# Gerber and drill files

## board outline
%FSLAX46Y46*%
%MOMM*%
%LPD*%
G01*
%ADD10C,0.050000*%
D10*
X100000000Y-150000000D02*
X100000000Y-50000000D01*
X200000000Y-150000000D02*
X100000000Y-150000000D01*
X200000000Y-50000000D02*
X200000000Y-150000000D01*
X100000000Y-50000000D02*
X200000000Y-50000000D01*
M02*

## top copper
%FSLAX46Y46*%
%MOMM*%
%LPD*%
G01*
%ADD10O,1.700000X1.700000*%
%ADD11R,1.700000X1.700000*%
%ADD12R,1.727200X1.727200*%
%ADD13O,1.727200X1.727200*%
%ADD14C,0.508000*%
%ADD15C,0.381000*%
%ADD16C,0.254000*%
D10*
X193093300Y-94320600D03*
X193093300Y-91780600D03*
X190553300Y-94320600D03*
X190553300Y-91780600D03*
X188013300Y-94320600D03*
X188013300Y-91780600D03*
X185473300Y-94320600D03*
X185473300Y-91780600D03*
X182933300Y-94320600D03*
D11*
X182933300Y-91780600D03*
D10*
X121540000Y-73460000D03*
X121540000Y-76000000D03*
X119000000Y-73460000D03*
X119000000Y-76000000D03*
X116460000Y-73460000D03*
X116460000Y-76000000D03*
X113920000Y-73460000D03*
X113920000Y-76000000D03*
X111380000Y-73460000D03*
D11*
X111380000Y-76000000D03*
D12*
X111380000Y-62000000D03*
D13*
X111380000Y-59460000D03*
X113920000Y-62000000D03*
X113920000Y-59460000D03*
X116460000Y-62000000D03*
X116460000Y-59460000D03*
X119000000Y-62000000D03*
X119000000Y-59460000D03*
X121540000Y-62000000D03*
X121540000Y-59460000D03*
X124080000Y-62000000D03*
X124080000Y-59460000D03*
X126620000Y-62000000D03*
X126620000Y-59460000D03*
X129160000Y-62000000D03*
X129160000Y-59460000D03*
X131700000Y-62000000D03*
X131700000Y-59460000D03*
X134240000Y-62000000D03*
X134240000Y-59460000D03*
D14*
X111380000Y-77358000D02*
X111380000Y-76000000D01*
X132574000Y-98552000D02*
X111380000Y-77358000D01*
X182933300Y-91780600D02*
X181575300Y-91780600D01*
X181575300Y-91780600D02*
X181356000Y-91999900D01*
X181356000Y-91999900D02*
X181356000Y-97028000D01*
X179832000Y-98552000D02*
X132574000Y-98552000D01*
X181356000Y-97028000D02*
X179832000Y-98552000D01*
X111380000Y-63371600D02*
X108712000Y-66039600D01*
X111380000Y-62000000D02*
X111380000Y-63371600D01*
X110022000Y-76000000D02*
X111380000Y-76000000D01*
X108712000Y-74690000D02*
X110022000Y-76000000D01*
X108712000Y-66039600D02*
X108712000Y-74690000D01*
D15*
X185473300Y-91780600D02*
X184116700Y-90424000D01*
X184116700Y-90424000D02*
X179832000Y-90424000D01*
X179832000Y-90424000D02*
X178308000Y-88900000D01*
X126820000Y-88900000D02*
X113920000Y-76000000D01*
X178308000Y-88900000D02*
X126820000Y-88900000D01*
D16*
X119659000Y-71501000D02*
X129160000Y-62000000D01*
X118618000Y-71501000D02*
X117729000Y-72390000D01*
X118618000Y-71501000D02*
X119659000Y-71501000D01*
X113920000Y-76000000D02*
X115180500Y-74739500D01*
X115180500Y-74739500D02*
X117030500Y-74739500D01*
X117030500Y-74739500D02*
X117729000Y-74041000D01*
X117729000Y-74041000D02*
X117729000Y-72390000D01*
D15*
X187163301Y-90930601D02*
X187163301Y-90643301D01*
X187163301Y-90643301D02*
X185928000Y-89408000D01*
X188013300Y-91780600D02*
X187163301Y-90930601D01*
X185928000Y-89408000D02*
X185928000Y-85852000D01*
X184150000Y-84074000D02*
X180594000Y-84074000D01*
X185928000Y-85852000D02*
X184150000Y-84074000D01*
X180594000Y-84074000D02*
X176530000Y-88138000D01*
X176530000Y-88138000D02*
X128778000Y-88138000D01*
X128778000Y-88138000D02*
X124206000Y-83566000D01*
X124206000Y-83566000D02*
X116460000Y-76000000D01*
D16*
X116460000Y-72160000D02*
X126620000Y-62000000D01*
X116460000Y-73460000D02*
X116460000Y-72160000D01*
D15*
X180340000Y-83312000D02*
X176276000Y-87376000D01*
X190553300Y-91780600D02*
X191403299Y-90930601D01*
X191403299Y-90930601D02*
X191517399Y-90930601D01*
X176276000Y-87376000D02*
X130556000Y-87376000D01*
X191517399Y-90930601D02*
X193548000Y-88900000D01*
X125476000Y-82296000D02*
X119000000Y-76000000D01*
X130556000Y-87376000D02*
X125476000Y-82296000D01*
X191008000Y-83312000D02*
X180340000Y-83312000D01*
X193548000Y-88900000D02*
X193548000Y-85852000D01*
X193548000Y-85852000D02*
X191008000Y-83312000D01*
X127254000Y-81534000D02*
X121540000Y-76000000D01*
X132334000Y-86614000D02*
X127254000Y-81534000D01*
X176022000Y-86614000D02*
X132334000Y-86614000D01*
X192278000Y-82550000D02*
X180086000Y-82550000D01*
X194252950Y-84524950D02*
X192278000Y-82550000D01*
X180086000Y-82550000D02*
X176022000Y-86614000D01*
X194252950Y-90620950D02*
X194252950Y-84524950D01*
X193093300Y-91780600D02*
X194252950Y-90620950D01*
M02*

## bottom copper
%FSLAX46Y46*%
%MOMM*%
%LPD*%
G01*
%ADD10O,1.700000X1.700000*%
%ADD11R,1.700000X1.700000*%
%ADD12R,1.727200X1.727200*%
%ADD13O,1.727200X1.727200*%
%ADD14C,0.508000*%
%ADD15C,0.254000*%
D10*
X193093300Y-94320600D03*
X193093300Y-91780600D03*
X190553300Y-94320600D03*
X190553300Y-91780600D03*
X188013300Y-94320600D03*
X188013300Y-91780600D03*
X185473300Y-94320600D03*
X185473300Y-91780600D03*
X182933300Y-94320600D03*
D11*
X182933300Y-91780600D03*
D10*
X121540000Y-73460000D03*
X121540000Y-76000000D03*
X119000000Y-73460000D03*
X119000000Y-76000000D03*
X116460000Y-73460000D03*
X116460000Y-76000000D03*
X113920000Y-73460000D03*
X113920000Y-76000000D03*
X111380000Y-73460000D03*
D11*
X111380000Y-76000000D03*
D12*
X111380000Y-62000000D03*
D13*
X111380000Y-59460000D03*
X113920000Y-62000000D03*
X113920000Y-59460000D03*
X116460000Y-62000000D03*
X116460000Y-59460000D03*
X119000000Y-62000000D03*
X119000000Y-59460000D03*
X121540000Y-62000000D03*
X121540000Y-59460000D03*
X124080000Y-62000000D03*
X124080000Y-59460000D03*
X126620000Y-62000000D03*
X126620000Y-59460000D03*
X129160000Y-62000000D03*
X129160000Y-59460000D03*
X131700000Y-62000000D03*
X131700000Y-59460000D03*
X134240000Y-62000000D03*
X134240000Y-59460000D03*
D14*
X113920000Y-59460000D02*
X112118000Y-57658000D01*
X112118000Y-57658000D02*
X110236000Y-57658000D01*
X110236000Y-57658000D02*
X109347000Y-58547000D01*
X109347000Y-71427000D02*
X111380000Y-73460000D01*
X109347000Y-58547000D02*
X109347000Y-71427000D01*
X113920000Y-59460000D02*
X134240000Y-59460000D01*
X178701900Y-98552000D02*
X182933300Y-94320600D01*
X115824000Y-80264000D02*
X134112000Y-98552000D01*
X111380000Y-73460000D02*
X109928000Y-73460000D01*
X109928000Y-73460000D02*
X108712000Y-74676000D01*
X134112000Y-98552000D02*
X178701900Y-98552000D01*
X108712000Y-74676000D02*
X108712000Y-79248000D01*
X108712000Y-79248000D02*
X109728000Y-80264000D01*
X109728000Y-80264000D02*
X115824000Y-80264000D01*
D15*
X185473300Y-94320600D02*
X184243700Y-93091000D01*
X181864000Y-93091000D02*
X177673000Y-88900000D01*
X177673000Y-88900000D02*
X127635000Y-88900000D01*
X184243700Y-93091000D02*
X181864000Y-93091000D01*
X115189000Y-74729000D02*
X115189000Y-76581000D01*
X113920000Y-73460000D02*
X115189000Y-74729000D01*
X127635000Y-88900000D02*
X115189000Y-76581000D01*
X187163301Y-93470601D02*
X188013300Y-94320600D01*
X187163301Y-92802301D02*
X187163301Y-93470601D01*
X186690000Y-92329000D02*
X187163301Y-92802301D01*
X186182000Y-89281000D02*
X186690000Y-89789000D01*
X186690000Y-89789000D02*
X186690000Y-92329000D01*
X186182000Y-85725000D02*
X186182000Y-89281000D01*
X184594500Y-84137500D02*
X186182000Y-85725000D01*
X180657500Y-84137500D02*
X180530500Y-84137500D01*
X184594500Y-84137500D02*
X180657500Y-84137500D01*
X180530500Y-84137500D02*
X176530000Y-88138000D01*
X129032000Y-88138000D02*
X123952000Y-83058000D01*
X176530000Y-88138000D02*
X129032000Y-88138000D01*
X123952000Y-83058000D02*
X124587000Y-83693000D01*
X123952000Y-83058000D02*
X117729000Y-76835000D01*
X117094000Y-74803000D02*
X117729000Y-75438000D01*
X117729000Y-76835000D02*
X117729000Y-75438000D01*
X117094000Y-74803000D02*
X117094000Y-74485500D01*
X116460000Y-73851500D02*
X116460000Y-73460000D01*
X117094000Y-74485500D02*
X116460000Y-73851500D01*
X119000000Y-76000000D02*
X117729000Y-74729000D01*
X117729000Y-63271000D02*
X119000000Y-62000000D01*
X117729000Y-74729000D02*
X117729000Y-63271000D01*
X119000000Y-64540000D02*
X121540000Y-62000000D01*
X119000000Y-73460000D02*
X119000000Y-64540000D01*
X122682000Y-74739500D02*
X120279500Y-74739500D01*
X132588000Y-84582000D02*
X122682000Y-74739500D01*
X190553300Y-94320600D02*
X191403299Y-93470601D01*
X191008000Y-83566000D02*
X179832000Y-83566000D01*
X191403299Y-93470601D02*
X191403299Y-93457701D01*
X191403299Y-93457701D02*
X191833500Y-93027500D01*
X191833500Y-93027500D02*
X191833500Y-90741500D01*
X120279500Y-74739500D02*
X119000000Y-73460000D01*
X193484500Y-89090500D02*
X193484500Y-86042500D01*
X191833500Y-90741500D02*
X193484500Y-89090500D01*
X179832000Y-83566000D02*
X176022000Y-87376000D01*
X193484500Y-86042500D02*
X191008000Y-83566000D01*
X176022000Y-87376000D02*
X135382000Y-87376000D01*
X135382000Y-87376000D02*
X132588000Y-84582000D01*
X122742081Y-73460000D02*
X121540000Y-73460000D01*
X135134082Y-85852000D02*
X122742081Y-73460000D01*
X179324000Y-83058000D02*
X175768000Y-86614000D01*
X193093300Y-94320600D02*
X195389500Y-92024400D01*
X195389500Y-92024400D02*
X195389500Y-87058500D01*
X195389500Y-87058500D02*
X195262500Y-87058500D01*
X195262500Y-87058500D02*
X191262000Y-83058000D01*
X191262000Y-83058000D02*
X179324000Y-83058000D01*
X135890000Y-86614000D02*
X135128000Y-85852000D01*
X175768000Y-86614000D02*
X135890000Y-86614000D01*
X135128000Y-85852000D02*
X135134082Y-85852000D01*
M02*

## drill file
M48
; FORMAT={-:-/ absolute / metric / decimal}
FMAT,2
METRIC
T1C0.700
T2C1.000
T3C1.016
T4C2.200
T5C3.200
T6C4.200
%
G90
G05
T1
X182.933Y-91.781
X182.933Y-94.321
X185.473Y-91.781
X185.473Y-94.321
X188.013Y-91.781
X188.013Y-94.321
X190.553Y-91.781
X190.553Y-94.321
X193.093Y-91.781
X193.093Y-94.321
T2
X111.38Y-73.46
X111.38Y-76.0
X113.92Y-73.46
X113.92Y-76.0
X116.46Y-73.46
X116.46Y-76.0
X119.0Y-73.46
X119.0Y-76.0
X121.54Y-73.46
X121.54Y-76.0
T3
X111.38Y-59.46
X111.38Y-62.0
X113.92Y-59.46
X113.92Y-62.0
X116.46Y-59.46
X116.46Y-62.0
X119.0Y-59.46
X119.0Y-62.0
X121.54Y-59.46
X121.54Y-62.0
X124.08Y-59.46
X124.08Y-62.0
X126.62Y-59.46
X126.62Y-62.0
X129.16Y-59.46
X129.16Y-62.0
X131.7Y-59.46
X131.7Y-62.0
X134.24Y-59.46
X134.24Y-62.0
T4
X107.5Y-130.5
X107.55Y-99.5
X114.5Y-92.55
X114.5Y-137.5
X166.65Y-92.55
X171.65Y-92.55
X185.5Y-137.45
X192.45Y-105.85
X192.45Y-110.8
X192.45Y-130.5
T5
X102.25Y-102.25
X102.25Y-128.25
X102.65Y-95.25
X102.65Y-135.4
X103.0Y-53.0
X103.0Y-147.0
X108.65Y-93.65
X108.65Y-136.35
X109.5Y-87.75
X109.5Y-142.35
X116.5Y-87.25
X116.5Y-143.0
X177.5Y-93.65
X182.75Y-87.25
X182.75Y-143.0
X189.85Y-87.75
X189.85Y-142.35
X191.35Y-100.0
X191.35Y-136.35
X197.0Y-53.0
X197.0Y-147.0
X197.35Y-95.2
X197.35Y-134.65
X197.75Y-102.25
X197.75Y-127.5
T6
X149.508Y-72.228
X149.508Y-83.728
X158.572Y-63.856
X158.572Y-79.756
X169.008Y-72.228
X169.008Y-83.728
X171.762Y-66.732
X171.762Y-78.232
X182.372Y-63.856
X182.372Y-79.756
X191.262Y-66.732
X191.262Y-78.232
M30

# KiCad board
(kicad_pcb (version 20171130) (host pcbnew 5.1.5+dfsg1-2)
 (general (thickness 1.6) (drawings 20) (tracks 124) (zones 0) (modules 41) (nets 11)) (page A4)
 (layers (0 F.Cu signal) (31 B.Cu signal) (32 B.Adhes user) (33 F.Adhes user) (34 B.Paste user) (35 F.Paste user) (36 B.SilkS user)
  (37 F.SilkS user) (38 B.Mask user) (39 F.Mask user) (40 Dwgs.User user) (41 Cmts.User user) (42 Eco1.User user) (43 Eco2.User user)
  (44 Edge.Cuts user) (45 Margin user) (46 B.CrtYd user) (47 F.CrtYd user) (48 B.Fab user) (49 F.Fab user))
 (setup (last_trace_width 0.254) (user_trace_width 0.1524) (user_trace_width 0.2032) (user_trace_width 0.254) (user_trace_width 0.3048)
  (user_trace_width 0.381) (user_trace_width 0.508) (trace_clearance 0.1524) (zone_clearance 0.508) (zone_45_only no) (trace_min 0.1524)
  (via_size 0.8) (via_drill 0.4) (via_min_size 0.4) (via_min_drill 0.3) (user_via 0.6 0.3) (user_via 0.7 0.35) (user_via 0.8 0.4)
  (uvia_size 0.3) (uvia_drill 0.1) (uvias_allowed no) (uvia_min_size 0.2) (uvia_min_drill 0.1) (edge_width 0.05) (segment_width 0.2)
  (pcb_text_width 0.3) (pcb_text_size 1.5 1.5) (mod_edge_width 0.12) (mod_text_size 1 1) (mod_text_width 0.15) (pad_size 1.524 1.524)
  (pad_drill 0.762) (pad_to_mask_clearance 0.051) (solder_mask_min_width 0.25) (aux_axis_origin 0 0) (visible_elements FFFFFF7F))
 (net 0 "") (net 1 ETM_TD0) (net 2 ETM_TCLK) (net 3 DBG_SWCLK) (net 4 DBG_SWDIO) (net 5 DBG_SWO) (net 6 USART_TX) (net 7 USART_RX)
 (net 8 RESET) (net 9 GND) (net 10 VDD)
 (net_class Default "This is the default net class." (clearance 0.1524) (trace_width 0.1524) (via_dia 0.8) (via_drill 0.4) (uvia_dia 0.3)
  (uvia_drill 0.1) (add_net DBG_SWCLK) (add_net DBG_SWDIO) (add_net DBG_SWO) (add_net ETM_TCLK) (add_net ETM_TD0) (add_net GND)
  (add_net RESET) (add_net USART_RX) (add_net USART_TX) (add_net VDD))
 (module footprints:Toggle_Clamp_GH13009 (layer F.Cu) (at 181.512 72.482)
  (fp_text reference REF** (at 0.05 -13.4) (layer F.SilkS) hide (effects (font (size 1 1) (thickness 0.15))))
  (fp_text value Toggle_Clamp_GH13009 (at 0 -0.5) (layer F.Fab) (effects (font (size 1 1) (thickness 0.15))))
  (pad "" np_thru_hole circle (at -9.75 -5.75) (size 4.2 4.2) (drill 4.2) (layers *.Cu *.Mask))
  (pad "" np_thru_hole circle (at -9.75 5.75) (size 4.2 4.2) (drill 4.2) (layers *.Cu *.Mask))
  (pad "" np_thru_hole circle (at 9.75 5.75) (size 4.2 4.2) (drill 4.2) (layers *.Cu *.Mask))
  (pad "" np_thru_hole circle (at 9.75 -5.75) (size 4.2 4.2) (drill 4.2) (layers *.Cu *.Mask)))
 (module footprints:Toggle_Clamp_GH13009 (layer F.Cu) (at 159.258 77.978)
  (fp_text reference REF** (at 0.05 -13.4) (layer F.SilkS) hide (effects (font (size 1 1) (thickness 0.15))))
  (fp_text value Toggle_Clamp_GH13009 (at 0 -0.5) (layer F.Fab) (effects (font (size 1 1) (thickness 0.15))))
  (pad "" np_thru_hole circle (at 9.75 -5.75) (size 4.2 4.2) (drill 4.2) (layers *.Cu *.Mask))
  (pad "" np_thru_hole circle (at 9.75 5.75) (size 4.2 4.2) (drill 4.2) (layers *.Cu *.Mask))
  (pad "" np_thru_hole circle (at -9.75 5.75) (size 4.2 4.2) (drill 4.2) (layers *.Cu *.Mask))
  (pad "" np_thru_hole circle (at -9.75 -5.75) (size 4.2 4.2) (drill 4.2) (layers *.Cu *.Mask)))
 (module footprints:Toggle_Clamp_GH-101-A (layer F.Cu) (at 170.472 71.806)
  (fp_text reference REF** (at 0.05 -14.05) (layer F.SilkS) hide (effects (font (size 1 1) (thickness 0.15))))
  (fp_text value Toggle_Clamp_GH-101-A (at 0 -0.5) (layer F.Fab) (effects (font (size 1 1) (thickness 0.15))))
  (pad "" np_thru_hole circle (at -11.9 -7.95) (size 4.2 4.2) (drill 4.2) (layers *.Cu *.Mask))
  (pad "" np_thru_hole circle (at -11.9 7.95) (size 4.2 4.2) (drill 4.2) (layers *.Cu *.Mask))
  (pad "" np_thru_hole circle (at 11.9 7.95) (size 4.2 4.2) (drill 4.2) (layers *.Cu *.Mask))
  (pad "" np_thru_hole circle (at 11.9 -7.95) (size 4.2 4.2) (drill 4.2) (layers *.Cu *.Mask)))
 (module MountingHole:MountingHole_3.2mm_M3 (layer F.Cu) (at 197 53)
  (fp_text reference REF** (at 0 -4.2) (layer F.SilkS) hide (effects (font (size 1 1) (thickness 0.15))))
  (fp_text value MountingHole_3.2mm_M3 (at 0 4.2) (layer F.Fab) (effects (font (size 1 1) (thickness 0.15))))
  (pad 1 np_thru_hole circle (at 0 0) (size 3.2 3.2) (drill 3.2) (layers *.Cu *.Mask)))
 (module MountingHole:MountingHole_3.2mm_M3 (layer F.Cu) (at 197 147)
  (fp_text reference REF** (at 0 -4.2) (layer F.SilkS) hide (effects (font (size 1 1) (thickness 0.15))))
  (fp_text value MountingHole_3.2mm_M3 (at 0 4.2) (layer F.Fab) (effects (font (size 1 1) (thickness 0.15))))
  (pad 1 np_thru_hole circle (at 0 0) (size 3.2 3.2) (drill 3.2) (layers *.Cu *.Mask)))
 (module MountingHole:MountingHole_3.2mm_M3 (layer F.Cu) (at 103 147)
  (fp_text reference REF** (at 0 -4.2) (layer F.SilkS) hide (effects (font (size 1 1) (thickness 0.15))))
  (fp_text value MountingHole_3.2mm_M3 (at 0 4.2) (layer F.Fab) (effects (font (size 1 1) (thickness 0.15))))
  (pad 1 np_thru_hole circle (at 0 0) (size 3.2 3.2) (drill 3.2) (layers *.Cu *.Mask)))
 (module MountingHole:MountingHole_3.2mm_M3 (layer F.Cu) (at 103 53)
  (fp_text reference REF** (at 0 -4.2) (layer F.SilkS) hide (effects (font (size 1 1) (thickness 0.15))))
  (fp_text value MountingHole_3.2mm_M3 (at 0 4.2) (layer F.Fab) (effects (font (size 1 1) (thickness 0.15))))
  (pad 1 np_thru_hole circle (at 0 0) (size 3.2 3.2) (drill 3.2) (layers *.Cu *.Mask)))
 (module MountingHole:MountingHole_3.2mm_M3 (layer F.Cu) (at 116.5 87.25)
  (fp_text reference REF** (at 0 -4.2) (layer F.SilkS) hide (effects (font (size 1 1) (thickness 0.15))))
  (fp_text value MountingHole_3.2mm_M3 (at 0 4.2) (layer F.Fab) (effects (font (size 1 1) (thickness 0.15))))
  (pad 1 np_thru_hole circle (at 0 0) (size 3.2 3.2) (drill 3.2) (layers *.Cu *.Mask)))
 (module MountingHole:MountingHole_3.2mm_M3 (layer F.Cu) (at 102.25 102.25)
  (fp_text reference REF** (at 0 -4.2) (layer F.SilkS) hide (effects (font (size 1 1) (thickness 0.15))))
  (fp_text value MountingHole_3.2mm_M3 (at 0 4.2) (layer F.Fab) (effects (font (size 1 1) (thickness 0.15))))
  (pad 1 np_thru_hole circle (at 0 0) (size 3.2 3.2) (drill 3.2) (layers *.Cu *.Mask)))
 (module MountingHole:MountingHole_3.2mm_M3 (layer F.Cu) (at 102.25 128.25)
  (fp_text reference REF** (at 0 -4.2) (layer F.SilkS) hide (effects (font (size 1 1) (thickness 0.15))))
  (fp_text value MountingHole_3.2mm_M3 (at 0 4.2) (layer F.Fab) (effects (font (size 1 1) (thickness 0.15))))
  (pad 1 np_thru_hole circle (at 0 0) (size 3.2 3.2) (drill 3.2) (layers *.Cu *.Mask)))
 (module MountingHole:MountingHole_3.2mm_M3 (layer F.Cu) (at 116.5 143)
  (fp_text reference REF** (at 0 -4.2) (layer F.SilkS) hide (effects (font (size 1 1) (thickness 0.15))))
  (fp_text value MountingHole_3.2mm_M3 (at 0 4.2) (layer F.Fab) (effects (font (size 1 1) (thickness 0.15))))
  (pad 1 np_thru_hole circle (at 0 0) (size 3.2 3.2) (drill 3.2) (layers *.Cu *.Mask)))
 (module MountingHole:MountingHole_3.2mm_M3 (layer F.Cu) (at 182.75 143)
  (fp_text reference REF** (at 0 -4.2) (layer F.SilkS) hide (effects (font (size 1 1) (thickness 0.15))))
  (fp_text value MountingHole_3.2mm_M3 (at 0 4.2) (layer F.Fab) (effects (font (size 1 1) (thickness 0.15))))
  (pad 1 np_thru_hole circle (at 0 0) (size 3.2 3.2) (drill 3.2) (layers *.Cu *.Mask)))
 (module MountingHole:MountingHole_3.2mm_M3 (layer F.Cu) (at 197.75 127.5)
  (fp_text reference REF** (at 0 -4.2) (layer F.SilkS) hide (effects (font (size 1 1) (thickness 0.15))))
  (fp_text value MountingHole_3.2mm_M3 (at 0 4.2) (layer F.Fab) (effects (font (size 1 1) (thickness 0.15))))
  (pad 1 np_thru_hole circle (at 0 0) (size 3.2 3.2) (drill 3.2) (layers *.Cu *.Mask)))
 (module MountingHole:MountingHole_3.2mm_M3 (layer F.Cu) (at 182.75 87.25)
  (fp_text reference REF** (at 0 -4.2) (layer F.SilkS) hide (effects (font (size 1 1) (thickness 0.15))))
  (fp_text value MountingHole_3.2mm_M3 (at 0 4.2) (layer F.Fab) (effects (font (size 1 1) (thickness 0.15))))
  (pad 1 np_thru_hole circle (at 0 0) (size 3.2 3.2) (drill 3.2) (layers *.Cu *.Mask)))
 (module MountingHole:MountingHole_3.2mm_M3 (layer F.Cu) (at 197.75 102.25)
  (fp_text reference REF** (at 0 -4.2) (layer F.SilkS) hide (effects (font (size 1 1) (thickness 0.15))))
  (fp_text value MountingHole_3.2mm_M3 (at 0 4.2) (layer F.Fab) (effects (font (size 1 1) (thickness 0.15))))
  (pad 1 np_thru_hole circle (at 0 0) (size 3.2 3.2) (drill 3.2) (layers *.Cu *.Mask)))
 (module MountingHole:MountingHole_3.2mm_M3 (layer F.Cu) (at 102.65 95.25)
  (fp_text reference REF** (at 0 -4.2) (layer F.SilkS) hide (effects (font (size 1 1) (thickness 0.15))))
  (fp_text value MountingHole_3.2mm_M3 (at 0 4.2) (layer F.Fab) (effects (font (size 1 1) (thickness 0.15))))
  (pad 1 np_thru_hole circle (at 0 0) (size 3.2 3.2) (drill 3.2) (layers *.Cu *.Mask)))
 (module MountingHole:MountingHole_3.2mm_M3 (layer F.Cu) (at 109.5 87.75)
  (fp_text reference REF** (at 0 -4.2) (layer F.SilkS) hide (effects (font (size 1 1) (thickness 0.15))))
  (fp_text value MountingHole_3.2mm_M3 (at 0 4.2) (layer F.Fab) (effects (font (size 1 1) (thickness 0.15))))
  (pad 1 np_thru_hole circle (at 0 0) (size 3.2 3.2) (drill 3.2) (layers *.Cu *.Mask)))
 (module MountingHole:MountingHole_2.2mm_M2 (layer F.Cu) (at 192.45 110.8)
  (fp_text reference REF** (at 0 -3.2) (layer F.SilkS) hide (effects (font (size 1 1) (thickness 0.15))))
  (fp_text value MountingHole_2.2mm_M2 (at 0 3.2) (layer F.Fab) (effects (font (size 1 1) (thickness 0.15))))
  (pad 1 np_thru_hole circle (at 0 0) (size 2.2 2.2) (drill 2.2) (layers *.Cu *.Mask)))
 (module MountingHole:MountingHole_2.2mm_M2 (layer F.Cu) (at 166.65 92.55)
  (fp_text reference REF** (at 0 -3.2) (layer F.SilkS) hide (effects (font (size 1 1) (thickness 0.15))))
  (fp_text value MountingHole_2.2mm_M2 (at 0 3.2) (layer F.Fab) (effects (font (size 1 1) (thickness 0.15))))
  (pad 1 np_thru_hole circle (at 0 0) (size 2.2 2.2) (drill 2.2) (layers *.Cu *.Mask)))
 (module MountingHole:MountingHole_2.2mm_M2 (layer F.Cu) (at 171.65 92.55)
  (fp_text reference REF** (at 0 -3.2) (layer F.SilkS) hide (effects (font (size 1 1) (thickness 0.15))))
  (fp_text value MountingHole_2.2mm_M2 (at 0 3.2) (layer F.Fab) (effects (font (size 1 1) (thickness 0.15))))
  (pad 1 np_thru_hole circle (at 0 0) (size 2.2 2.2) (drill 2.2) (layers *.Cu *.Mask)))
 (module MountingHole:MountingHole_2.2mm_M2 (layer F.Cu) (at 192.45 105.85)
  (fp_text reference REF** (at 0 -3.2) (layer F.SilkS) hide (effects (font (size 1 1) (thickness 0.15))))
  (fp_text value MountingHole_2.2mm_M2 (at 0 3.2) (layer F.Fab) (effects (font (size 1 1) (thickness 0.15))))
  (pad 1 np_thru_hole circle (at 0 0) (size 2.2 2.2) (drill 2.2) (layers *.Cu *.Mask)))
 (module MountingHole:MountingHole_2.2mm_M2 (layer F.Cu) (at 192.45 130.5)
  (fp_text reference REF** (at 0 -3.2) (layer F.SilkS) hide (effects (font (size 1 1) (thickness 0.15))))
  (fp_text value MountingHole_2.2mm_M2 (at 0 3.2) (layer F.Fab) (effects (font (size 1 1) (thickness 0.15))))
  (pad 1 np_thru_hole circle (at 0 0) (size 2.2 2.2) (drill 2.2) (layers *.Cu *.Mask)))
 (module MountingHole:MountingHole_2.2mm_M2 (layer F.Cu) (at 185.5 137.45)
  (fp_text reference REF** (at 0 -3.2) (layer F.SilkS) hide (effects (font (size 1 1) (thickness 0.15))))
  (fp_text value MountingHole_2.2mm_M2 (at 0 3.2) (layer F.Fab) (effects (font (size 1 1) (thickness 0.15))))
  (pad 1 np_thru_hole circle (at 0 0) (size 2.2 2.2) (drill 2.2) (layers *.Cu *.Mask)))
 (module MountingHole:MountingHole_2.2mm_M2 (layer F.Cu) (at 107.5 130.5)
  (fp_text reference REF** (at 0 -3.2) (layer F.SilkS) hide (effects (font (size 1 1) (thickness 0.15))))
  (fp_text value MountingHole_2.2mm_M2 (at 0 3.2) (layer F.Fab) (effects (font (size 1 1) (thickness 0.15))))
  (pad 1 np_thru_hole circle (at 0 0) (size 2.2 2.2) (drill 2.2) (layers *.Cu *.Mask)))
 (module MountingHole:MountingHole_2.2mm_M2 (layer F.Cu) (at 114.5 137.5)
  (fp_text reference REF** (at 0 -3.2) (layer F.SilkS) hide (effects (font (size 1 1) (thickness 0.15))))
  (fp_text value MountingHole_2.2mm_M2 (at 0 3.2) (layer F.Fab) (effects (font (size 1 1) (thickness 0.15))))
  (pad 1 np_thru_hole circle (at 0 0) (size 2.2 2.2) (drill 2.2) (layers *.Cu *.Mask)))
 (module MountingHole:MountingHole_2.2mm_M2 (layer F.Cu) (at 114.5 92.55)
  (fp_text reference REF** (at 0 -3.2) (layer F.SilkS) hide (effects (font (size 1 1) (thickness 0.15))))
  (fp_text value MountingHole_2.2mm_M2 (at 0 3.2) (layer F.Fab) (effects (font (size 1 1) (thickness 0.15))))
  (pad 1 np_thru_hole circle (at 0 0) (size 2.2 2.2) (drill 2.2) (layers *.Cu *.Mask)))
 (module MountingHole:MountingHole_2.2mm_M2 (layer F.Cu) (at 107.55 99.5)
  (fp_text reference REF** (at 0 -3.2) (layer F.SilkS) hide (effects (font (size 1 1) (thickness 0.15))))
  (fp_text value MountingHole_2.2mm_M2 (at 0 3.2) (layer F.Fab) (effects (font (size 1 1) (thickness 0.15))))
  (pad 1 np_thru_hole circle (at 0 0) (size 2.2 2.2) (drill 2.2) (layers *.Cu *.Mask)))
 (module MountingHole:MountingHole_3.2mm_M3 (layer F.Cu) (at 197.35 95.2)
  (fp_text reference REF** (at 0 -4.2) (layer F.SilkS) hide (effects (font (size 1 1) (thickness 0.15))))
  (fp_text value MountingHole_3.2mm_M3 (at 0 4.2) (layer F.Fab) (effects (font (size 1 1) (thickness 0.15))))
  (pad 1 np_thru_hole circle (at 0 0) (size 3.2 3.2) (drill 3.2) (layers *.Cu *.Mask)))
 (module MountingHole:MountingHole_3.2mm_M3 (layer F.Cu) (at 189.85 87.75)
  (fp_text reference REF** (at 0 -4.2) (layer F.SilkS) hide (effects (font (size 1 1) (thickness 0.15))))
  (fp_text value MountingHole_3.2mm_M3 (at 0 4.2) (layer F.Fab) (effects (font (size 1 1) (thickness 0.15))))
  (pad 1 np_thru_hole circle (at 0 0) (size 3.2 3.2) (drill 3.2) (layers *.Cu *.Mask)))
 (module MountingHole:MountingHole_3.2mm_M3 (layer F.Cu) (at 197.35 134.65)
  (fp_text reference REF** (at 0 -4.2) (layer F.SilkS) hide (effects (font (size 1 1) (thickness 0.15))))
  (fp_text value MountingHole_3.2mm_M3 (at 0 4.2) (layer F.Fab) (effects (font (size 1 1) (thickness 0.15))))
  (pad 1 np_thru_hole circle (at 0 0) (size 3.2 3.2) (drill 3.2) (layers *.Cu *.Mask)))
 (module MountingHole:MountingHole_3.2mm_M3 (layer F.Cu) (at 189.85 142.35)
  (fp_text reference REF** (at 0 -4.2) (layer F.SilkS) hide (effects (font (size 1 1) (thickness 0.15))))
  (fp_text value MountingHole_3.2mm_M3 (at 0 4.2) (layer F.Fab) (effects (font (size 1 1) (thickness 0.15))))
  (pad 1 np_thru_hole circle (at 0 0) (size 3.2 3.2) (drill 3.2) (layers *.Cu *.Mask)))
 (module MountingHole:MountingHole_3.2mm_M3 (layer F.Cu) (at 109.5 142.35)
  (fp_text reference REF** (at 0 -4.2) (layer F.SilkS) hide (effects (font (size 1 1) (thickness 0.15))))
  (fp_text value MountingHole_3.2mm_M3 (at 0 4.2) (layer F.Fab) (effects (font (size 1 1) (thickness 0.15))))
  (pad 1 np_thru_hole circle (at 0 0) (size 3.2 3.2) (drill 3.2) (layers *.Cu *.Mask)))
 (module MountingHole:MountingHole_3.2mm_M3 (layer F.Cu) (at 191.35 100)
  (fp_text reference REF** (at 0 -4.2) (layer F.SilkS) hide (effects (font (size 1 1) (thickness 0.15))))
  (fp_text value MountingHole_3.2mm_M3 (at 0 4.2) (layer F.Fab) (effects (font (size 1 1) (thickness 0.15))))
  (pad 1 np_thru_hole circle (at 0 0) (size 3.2 3.2) (drill 3.2) (layers *.Cu *.Mask)))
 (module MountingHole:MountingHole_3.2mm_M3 (layer F.Cu) (at 191.35 136.35)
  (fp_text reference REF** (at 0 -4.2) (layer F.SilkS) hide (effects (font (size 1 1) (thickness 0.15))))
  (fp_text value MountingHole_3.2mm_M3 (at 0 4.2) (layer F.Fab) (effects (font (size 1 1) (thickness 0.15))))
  (pad 1 np_thru_hole circle (at 0 0) (size 3.2 3.2) (drill 3.2) (layers *.Cu *.Mask)))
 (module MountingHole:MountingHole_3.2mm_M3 (layer F.Cu) (at 177.5 93.65)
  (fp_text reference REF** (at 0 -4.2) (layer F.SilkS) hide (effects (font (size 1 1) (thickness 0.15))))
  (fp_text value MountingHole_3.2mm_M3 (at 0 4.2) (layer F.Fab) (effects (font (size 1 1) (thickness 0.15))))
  (pad 1 np_thru_hole circle (at 0 0) (size 3.2 3.2) (drill 3.2) (layers *.Cu *.Mask)))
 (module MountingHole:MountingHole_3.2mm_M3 (layer F.Cu) (at 108.65 93.65)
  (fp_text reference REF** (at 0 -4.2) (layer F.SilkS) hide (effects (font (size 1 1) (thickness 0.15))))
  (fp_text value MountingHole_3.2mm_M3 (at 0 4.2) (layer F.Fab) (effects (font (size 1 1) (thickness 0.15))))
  (pad 1 np_thru_hole circle (at 0 0) (size 3.2 3.2) (drill 3.2) (layers *.Cu *.Mask)))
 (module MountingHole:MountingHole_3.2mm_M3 (layer F.Cu) (at 102.65 135.4)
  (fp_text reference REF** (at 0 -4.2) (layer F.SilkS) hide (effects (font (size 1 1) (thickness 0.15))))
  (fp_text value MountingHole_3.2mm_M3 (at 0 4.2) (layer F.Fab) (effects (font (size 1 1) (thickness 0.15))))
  (pad 1 np_thru_hole circle (at 0 0) (size 3.2 3.2) (drill 3.2) (layers *.Cu *.Mask)))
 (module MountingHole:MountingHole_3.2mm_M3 (layer F.Cu) (at 108.65 136.35)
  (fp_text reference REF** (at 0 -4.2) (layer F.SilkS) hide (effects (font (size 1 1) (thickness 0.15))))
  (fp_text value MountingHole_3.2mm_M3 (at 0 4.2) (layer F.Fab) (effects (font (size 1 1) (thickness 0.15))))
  (pad 1 np_thru_hole circle (at 0 0) (size 3.2 3.2) (drill 3.2) (layers *.Cu *.Mask)))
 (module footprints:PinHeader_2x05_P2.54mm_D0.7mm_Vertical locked (layer F.Cu) (at 182.9333 94.3206 90)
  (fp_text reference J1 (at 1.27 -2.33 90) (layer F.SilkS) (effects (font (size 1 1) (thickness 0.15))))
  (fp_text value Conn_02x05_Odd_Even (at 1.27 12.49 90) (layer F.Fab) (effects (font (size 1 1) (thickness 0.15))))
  (pad 10 thru_hole oval (at 0 10.16 90) (size 1.7 1.7) (drill 0.7) (layers *.Cu *.Mask) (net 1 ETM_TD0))
  (pad 9 thru_hole oval (at 2.54 10.16 90) (size 1.7 1.7) (drill 0.7) (layers *.Cu *.Mask) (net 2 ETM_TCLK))
  (pad 8 thru_hole oval (at 0 7.62 90) (size 1.7 1.7) (drill 0.7) (layers *.Cu *.Mask) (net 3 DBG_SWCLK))
  (pad 7 thru_hole oval (at 2.54 7.62 90) (size 1.7 1.7) (drill 0.7) (layers *.Cu *.Mask) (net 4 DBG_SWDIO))
  (pad 6 thru_hole oval (at 0 5.08 90) (size 1.7 1.7) (drill 0.7) (layers *.Cu *.Mask) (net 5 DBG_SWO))
  (pad 5 thru_hole oval (at 2.54 5.08 90) (size 1.7 1.7) (drill 0.7) (layers *.Cu *.Mask) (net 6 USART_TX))
  (pad 4 thru_hole oval (at 0 2.54 90) (size 1.7 1.7) (drill 0.7) (layers *.Cu *.Mask) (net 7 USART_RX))
  (pad 3 thru_hole oval (at 2.54 2.54 90) (size 1.7 1.7) (drill 0.7) (layers *.Cu *.Mask) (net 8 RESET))
  (pad 2 thru_hole oval (at 0 0 90) (size 1.7 1.7) (drill 0.7) (layers *.Cu *.Mask) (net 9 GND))
  (pad 1 thru_hole rect (at 2.54 0 90) (size 1.7 1.7) (drill 0.7) (layers *.Cu *.Mask) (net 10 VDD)))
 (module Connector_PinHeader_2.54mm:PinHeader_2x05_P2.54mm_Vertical (layer F.Cu) (at 111.38 76 90)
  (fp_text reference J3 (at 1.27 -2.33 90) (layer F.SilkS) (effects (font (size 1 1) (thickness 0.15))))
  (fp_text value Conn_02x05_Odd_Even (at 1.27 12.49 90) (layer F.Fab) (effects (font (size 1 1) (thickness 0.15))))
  (pad 10 thru_hole oval (at 2.54 10.16 90) (size 1.7 1.7) (drill 1) (layers *.Cu *.Mask) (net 1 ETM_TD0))
  (pad 9 thru_hole oval (at 0 10.16 90) (size 1.7 1.7) (drill 1) (layers *.Cu *.Mask) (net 2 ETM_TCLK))
  (pad 8 thru_hole oval (at 2.54 7.62 90) (size 1.7 1.7) (drill 1) (layers *.Cu *.Mask) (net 3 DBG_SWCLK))
  (pad 7 thru_hole oval (at 0 7.62 90) (size 1.7 1.7) (drill 1) (layers *.Cu *.Mask) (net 4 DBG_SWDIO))
  (pad 6 thru_hole oval (at 2.54 5.08 90) (size 1.7 1.7) (drill 1) (layers *.Cu *.Mask) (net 5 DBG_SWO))
  (pad 5 thru_hole oval (at 0 5.08 90) (size 1.7 1.7) (drill 1) (layers *.Cu *.Mask) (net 6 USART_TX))
  (pad 4 thru_hole oval (at 2.54 2.54 90) (size 1.7 1.7) (drill 1) (layers *.Cu *.Mask) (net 7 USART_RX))
  (pad 3 thru_hole oval (at 0 2.54 90) (size 1.7 1.7) (drill 1) (layers *.Cu *.Mask) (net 8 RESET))
  (pad 2 thru_hole oval (at 2.54 0 90) (size 1.7 1.7) (drill 1) (layers *.Cu *.Mask) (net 9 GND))
  (pad 1 thru_hole rect (at 0 0 90) (size 1.7 1.7) (drill 1) (layers *.Cu *.Mask) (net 10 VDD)))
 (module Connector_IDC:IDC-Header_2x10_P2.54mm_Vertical (layer F.Cu) (at 111.38 62 90)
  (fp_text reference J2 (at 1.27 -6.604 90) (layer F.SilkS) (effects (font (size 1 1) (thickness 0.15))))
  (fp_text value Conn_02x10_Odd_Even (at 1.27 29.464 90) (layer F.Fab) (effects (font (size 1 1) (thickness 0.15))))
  (pad 1 thru_hole rect (at 0 0 90) (size 1.7272 1.7272) (drill 1.016) (layers *.Cu *.Mask) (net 10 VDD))
  (pad 2 thru_hole oval (at 2.54 0 90) (size 1.7272 1.7272) (drill 1.016) (layers *.Cu *.Mask))
  (pad 3 thru_hole oval (at 0 2.54 90) (size 1.7272 1.7272) (drill 1.016) (layers *.Cu *.Mask))
  (pad 4 thru_hole oval (at 2.54 2.54 90) (size 1.7272 1.7272) (drill 1.016) (layers *.Cu *.Mask) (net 9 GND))
  (pad 5 thru_hole oval (at 0 5.08 90) (size 1.7272 1.7272) (drill 1.016) (layers *.Cu *.Mask))
  (pad 6 thru_hole oval (at 2.54 5.08 90) (size 1.7272 1.7272) (drill 1.016) (layers *.Cu *.Mask) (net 9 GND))
  (pad 7 thru_hole oval (at 0 7.62 90) (size 1.7272 1.7272) (drill 1.016) (layers *.Cu *.Mask) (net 4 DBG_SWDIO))
  (pad 8 thru_hole oval (at 2.54 7.62 90) (size 1.7272 1.7272) (drill 1.016) (layers *.Cu *.Mask) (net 9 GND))
  (pad 9 thru_hole oval (at 0 10.16 90) (size 1.7272 1.7272) (drill 1.016) (layers *.Cu *.Mask) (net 3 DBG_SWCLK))
  (pad 10 thru_hole oval (at 2.54 10.16 90) (size 1.7272 1.7272) (drill 1.016) (layers *.Cu *.Mask) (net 9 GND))
  (pad 11 thru_hole oval (at 0 12.7 90) (size 1.7272 1.7272) (drill 1.016) (layers *.Cu *.Mask))
  (pad 12 thru_hole oval (at 2.54 12.7 90) (size 1.7272 1.7272) (drill 1.016) (layers *.Cu *.Mask) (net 9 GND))
  (pad 13 thru_hole oval (at 0 15.24 90) (size 1.7272 1.7272) (drill 1.016) (layers *.Cu *.Mask) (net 5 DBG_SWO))
  (pad 14 thru_hole oval (at 2.54 15.24 90) (size 1.7272 1.7272) (drill 1.016) (layers *.Cu *.Mask) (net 9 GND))
  (pad 15 thru_hole oval (at 0 17.78 90) (size 1.7272 1.7272) (drill 1.016) (layers *.Cu *.Mask) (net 8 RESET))
  (pad 16 thru_hole oval (at 2.54 17.78 90) (size 1.7272 1.7272) (drill 1.016) (layers *.Cu *.Mask) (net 9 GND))
  (pad 17 thru_hole oval (at 0 20.32 90) (size 1.7272 1.7272) (drill 1.016) (layers *.Cu *.Mask))
  (pad 18 thru_hole oval (at 2.54 20.32 90) (size 1.7272 1.7272) (drill 1.016) (layers *.Cu *.Mask) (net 9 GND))
  (pad 19 thru_hole oval (at 0 22.86 90) (size 1.7272 1.7272) (drill 1.016) (layers *.Cu *.Mask))
  (pad 20 thru_hole oval (at 2.54 22.86 90) (size 1.7272 1.7272) (drill 1.016) (layers *.Cu *.Mask) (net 9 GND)))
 (gr_line (start 100 150) (end 100 50) (layer Edge.Cuts) (width 0.05))
 (gr_line (start 200 150) (end 100 150) (layer Edge.Cuts) (width 0.05))
 (gr_line (start 200 50) (end 200 150) (layer Edge.Cuts) (width 0.05))
 (gr_line (start 100 50) (end 200 50) (layer Edge.Cuts) (width 0.05))
 (segment (start 111.38 77.358) (end 111.38 76) (width 0.508) (layer F.Cu) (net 10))
 (segment (start 132.574 98.552) (end 111.38 77.358) (width 0.508) (layer F.Cu) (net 10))
 (segment (start 182.9333 91.7806) (end 181.5753 91.7806) (width 0.508) (layer F.Cu) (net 10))
 (segment (start 181.5753 91.7806) (end 181.356 91.9999) (width 0.508) (layer F.Cu) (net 10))
 (segment (start 181.356 91.9999) (end 181.356 97.028) (width 0.508) (layer F.Cu) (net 10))
 (segment (start 179.832 98.552) (end 132.574 98.552) (width 0.508) (layer F.Cu) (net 10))
 (segment (start 181.356 97.028) (end 179.832 98.552) (width 0.508) (layer F.Cu) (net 10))
 (segment (start 111.38 63.3716) (end 108.712 66.0396) (width 0.508) (layer F.Cu) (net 10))
 (segment (start 111.38 62) (end 111.38 63.3716) (width 0.508) (layer F.Cu) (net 10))
 (segment (start 110.022 76) (end 111.38 76) (width 0.508) (layer F.Cu) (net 10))
 (segment (start 108.712 74.69) (end 110.022 76) (width 0.508) (layer F.Cu) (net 10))
 (segment (start 108.712 66.0396) (end 108.712 74.69) (width 0.508) (layer F.Cu) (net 10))
 (segment (start 113.92 59.46) (end 112.118 57.658) (width 0.508) (layer B.Cu) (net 9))
 (segment (start 112.118 57.658) (end 110.236 57.658) (width 0.508) (layer B.Cu) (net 9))
 (segment (start 110.236 57.658) (end 109.347 58.547) (width 0.508) (layer B.Cu) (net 9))
 (segment (start 109.347 71.427) (end 111.38 73.46) (width 0.508) (layer B.Cu) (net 9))
 (segment (start 109.347 58.547) (end 109.347 71.427) (width 0.508) (layer B.Cu) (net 9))
 (segment (start 113.92 59.46) (end 134.24 59.46) (width 0.508) (layer B.Cu) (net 9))
 (segment (start 178.7019 98.552) (end 182.9333 94.3206) (width 0.508) (layer B.Cu) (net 9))
 (segment (start 115.824 80.264) (end 134.112 98.552) (width 0.508) (layer B.Cu) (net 9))
 (segment (start 111.38 73.46) (end 109.928 73.46) (width 0.508) (layer B.Cu) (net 9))
 (segment (start 109.928 73.46) (end 108.712 74.676) (width 0.508) (layer B.Cu) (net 9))
 (segment (start 134.112 98.552) (end 178.7019 98.552) (width 0.508) (layer B.Cu) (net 9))
 (segment (start 108.712 74.676) (end 108.712 79.248) (width 0.508) (layer B.Cu) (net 9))
 (segment (start 108.712 79.248) (end 109.728 80.264) (width 0.508) (layer B.Cu) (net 9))
 (segment (start 109.728 80.264) (end 115.824 80.264) (width 0.508) (layer B.Cu) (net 9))
 (segment (start 185.4733 91.7806) (end 184.1167 90.424) (width 0.381) (layer F.Cu) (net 8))
 (segment (start 184.1167 90.424) (end 179.832 90.424) (width 0.381) (layer F.Cu) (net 8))
 (segment (start 179.832 90.424) (end 178.308 88.9) (width 0.381) (layer F.Cu) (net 8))
 (segment (start 126.82 88.9) (end 113.92 76) (width 0.381) (layer F.Cu) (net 8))
 (segment (start 178.308 88.9) (end 126.82 88.9) (width 0.381) (layer F.Cu) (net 8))
 (segment (start 119.659 71.501) (end 129.16 62) (width 0.254) (layer F.Cu) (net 8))
 (segment (start 118.618 71.501) (end 117.729 72.39) (width 0.254) (layer F.Cu) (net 8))
 (segment (start 118.618 71.501) (end 119.659 71.501) (width 0.254) (layer F.Cu) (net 8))
 (segment (start 113.92 76) (end 115.1805 74.7395) (width 0.254) (layer F.Cu) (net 8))
 (segment (start 115.1805 74.7395) (end 117.0305 74.7395) (width 0.254) (layer F.Cu) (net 8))
 (segment (start 117.0305 74.7395) (end 117.729 74.041) (width 0.254) (layer F.Cu) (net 8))
 (segment (start 117.729 74.041) (end 117.729 72.39) (width 0.254) (layer F.Cu) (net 8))
 (segment (start 185.4733 94.3206) (end 184.2437 93.091) (width 0.254) (layer B.Cu) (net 7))
 (segment (start 181.864 93.091) (end 177.673 88.9) (width 0.254) (layer B.Cu) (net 7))
 (segment (start 177.673 88.9) (end 127.635 88.9) (width 0.254) (layer B.Cu) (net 7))
 (segment (start 184.2437 93.091) (end 181.864 93.091) (width 0.254) (layer B.Cu) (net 7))
 (segment (start 115.189 74.729) (end 115.189 76.581) (width 0.254) (layer B.Cu) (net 7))
 (segment (start 113.92 73.46) (end 115.189 74.729) (width 0.254) (layer B.Cu) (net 7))
 (segment (start 127.635 88.9) (end 115.189 76.581) (width 0.254) (layer B.Cu) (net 7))
 (segment (start 187.163301 90.930601) (end 187.163301 90.643301) (width 0.381) (layer F.Cu) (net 6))
 (segment (start 187.163301 90.643301) (end 185.928 89.408) (width 0.381) (layer F.Cu) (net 6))
 (segment (start 188.0133 91.7806) (end 187.163301 90.930601) (width 0.381) (layer F.Cu) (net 6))
 (segment (start 185.928 89.408) (end 185.928 85.852) (width 0.381) (layer F.Cu) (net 6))
 (segment (start 184.15 84.074) (end 180.594 84.074) (width 0.381) (layer F.Cu) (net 6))
 (segment (start 185.928 85.852) (end 184.15 84.074) (width 0.381) (layer F.Cu) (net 6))
 (segment (start 180.594 84.074) (end 176.53 88.138) (width 0.381) (layer F.Cu) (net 6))
 (segment (start 176.53 88.138) (end 128.778 88.138) (width 0.381) (layer F.Cu) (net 6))
 (segment (start 128.778 88.138) (end 124.206 83.566) (width 0.381) (layer F.Cu) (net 6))
 (segment (start 124.206 83.566) (end 116.46 76) (width 0.381) (layer F.Cu) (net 6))
 (segment (start 116.46 72.16) (end 126.62 62) (width 0.254) (layer F.Cu) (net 5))
 (segment (start 116.46 73.46) (end 116.46 72.16) (width 0.254) (layer F.Cu) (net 5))
 (segment (start 187.163301 93.470601) (end 188.0133 94.3206) (width 0.254) (layer B.Cu) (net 5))
 (segment (start 187.163301 92.802301) (end 187.163301 93.470601) (width 0.254) (layer B.Cu) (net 5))
 (segment (start 186.69 92.329) (end 187.163301 92.802301) (width 0.254) (layer B.Cu) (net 5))
 (segment (start 186.182 89.281) (end 186.69 89.789) (width 0.254) (layer B.Cu) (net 5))
 (segment (start 186.69 89.789) (end 186.69 92.329) (width 0.254) (layer B.Cu) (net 5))
 (segment (start 186.182 85.725) (end 186.182 89.281) (width 0.254) (layer B.Cu) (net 5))
 (segment (start 184.5945 84.1375) (end 186.182 85.725) (width 0.254) (layer B.Cu) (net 5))
 (segment (start 180.6575 84.1375) (end 180.5305 84.1375) (width 0.254) (layer B.Cu) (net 5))
 (segment (start 184.5945 84.1375) (end 180.6575 84.1375) (width 0.254) (layer B.Cu) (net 5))
 (segment (start 180.5305 84.1375) (end 176.53 88.138) (width 0.254) (layer B.Cu) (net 5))
 (segment (start 129.032 88.138) (end 123.952 83.058) (width 0.254) (layer B.Cu) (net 5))
 (segment (start 176.53 88.138) (end 129.032 88.138) (width 0.254) (layer B.Cu) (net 5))
 (segment (start 123.952 83.058) (end 124.587 83.693) (width 0.254) (layer B.Cu) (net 5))
 (segment (start 123.952 83.058) (end 117.729 76.835) (width 0.254) (layer B.Cu) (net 5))
 (segment (start 117.094 74.803) (end 117.729 75.438) (width 0.254) (layer B.Cu) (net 5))
 (segment (start 117.729 76.835) (end 117.729 75.438) (width 0.254) (layer B.Cu) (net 5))
 (segment (start 117.094 74.803) (end 117.094 74.4855) (width 0.254) (layer B.Cu) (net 5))
 (segment (start 116.46 73.8515) (end 116.46 73.46) (width 0.254) (layer B.Cu) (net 5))
 (segment (start 117.094 74.4855) (end 116.46 73.8515) (width 0.254) (layer B.Cu) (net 5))
 (segment (start 119 76) (end 117.729 74.729) (width 0.254) (layer B.Cu) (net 4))
 (segment (start 117.729 63.271) (end 119 62) (width 0.254) (layer B.Cu) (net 4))
 (segment (start 117.729 74.729) (end 117.729 63.271) (width 0.254) (layer B.Cu) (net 4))
 (segment (start 180.34 83.312) (end 176.276 87.376) (width 0.381) (layer F.Cu) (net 4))
 (segment (start 190.5533 91.7806) (end 191.403299 90.930601) (width 0.381) (layer F.Cu) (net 4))
 (segment (start 191.403299 90.930601) (end 191.517399 90.930601) (width 0.381) (layer F.Cu) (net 4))
 (segment (start 176.276 87.376) (end 130.556 87.376) (width 0.381) (layer F.Cu) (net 4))
 (segment (start 191.517399 90.930601) (end 193.548 88.9) (width 0.381) (layer F.Cu) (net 4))
 (segment (start 125.476 82.296) (end 119 76) (width 0.381) (layer F.Cu) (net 4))
 (segment (start 130.556 87.376) (end 125.476 82.296) (width 0.381) (layer F.Cu) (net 4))
 (segment (start 191.008 83.312) (end 180.34 83.312) (width 0.381) (layer F.Cu) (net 4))
 (segment (start 193.548 88.9) (end 193.548 85.852) (width 0.381) (layer F.Cu) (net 4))
 (segment (start 193.548 85.852) (end 191.008 83.312) (width 0.381) (layer F.Cu) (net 4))
 (segment (start 119 64.54) (end 121.54 62) (width 0.254) (layer B.Cu) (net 3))
 (segment (start 119 73.46) (end 119 64.54) (width 0.254) (layer B.Cu) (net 3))
 (segment (start 122.682 74.7395) (end 120.2795 74.7395) (width 0.254) (layer B.Cu) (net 3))
 (segment (start 132.588 84.582) (end 122.682 74.7395) (width 0.254) (layer B.Cu) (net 3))
 (segment (start 190.5533 94.3206) (end 191.403299 93.470601) (width 0.254) (layer B.Cu) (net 3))
 (segment (start 191.008 83.566) (end 179.832 83.566) (width 0.254) (layer B.Cu) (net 3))
 (segment (start 191.403299 93.470601) (end 191.403299 93.457701) (width 0.254) (layer B.Cu) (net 3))
 (segment (start 191.403299 93.457701) (end 191.8335 93.0275) (width 0.254) (layer B.Cu) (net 3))
 (segment (start 191.8335 93.0275) (end 191.8335 90.7415) (width 0.254) (layer B.Cu) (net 3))
 (segment (start 120.2795 74.7395) (end 119 73.46) (width 0.254) (layer B.Cu) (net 3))
 (segment (start 193.4845 89.0905) (end 193.4845 86.0425) (width 0.254) (layer B.Cu) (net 3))
 (segment (start 191.8335 90.7415) (end 193.4845 89.0905) (width 0.254) (layer B.Cu) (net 3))
 (segment (start 179.832 83.566) (end 176.022 87.376) (width 0.254) (layer B.Cu) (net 3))
 (segment (start 193.4845 86.0425) (end 191.008 83.566) (width 0.254) (layer B.Cu) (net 3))
 (segment (start 176.022 87.376) (end 135.382 87.376) (width 0.254) (layer B.Cu) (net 3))
 (segment (start 135.382 87.376) (end 132.588 84.582) (width 0.254) (layer B.Cu) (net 3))
 (segment (start 127.254 81.534) (end 121.54 76) (width 0.381) (layer F.Cu) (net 2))
 (segment (start 132.334 86.614) (end 127.254 81.534) (width 0.381) (layer F.Cu) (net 2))
 (segment (start 176.022 86.614) (end 132.334 86.614) (width 0.381) (layer F.Cu) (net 2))
 (segment (start 192.278 82.55) (end 180.086 82.55) (width 0.381) (layer F.Cu) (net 2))
 (segment (start 194.25295 84.52495) (end 192.278 82.55) (width 0.381) (layer F.Cu) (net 2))
 (segment (start 180.086 82.55) (end 176.022 86.614) (width 0.381) (layer F.Cu) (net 2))
 (segment (start 194.25295 90.62095) (end 194.25295 84.52495) (width 0.381) (layer F.Cu) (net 2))
 (segment (start 193.0933 91.7806) (end 194.25295 90.62095) (width 0.381) (layer F.Cu) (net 2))
 (segment (start 122.742081 73.46) (end 121.54 73.46) (width 0.254) (layer B.Cu) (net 1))
 (segment (start 135.134082 85.852) (end 122.742081 73.46) (width 0.254) (layer B.Cu) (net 1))
 (segment (start 179.324 83.058) (end 175.768 86.614) (width 0.254) (layer B.Cu) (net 1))
 (segment (start 193.0933 94.3206) (end 195.3895 92.0244) (width 0.254) (layer B.Cu) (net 1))
 (segment (start 195.3895 92.0244) (end 195.3895 87.0585) (width 0.254) (layer B.Cu) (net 1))
 (segment (start 195.3895 87.0585) (end 195.2625 87.0585) (width 0.254) (layer B.Cu) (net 1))
 (segment (start 195.2625 87.0585) (end 191.262 83.058) (width 0.254) (layer B.Cu) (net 1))
 (segment (start 191.262 83.058) (end 179.324 83.058) (width 0.254) (layer B.Cu) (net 1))
 (segment (start 135.89 86.614) (end 135.128 85.852) (width 0.254) (layer B.Cu) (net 1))
 (segment (start 175.768 86.614) (end 135.89 86.614) (width 0.254) (layer B.Cu) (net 1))
 (segment (start 135.128 85.852) (end 135.134082 85.852) (width 0.254) (layer B.Cu) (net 1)))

